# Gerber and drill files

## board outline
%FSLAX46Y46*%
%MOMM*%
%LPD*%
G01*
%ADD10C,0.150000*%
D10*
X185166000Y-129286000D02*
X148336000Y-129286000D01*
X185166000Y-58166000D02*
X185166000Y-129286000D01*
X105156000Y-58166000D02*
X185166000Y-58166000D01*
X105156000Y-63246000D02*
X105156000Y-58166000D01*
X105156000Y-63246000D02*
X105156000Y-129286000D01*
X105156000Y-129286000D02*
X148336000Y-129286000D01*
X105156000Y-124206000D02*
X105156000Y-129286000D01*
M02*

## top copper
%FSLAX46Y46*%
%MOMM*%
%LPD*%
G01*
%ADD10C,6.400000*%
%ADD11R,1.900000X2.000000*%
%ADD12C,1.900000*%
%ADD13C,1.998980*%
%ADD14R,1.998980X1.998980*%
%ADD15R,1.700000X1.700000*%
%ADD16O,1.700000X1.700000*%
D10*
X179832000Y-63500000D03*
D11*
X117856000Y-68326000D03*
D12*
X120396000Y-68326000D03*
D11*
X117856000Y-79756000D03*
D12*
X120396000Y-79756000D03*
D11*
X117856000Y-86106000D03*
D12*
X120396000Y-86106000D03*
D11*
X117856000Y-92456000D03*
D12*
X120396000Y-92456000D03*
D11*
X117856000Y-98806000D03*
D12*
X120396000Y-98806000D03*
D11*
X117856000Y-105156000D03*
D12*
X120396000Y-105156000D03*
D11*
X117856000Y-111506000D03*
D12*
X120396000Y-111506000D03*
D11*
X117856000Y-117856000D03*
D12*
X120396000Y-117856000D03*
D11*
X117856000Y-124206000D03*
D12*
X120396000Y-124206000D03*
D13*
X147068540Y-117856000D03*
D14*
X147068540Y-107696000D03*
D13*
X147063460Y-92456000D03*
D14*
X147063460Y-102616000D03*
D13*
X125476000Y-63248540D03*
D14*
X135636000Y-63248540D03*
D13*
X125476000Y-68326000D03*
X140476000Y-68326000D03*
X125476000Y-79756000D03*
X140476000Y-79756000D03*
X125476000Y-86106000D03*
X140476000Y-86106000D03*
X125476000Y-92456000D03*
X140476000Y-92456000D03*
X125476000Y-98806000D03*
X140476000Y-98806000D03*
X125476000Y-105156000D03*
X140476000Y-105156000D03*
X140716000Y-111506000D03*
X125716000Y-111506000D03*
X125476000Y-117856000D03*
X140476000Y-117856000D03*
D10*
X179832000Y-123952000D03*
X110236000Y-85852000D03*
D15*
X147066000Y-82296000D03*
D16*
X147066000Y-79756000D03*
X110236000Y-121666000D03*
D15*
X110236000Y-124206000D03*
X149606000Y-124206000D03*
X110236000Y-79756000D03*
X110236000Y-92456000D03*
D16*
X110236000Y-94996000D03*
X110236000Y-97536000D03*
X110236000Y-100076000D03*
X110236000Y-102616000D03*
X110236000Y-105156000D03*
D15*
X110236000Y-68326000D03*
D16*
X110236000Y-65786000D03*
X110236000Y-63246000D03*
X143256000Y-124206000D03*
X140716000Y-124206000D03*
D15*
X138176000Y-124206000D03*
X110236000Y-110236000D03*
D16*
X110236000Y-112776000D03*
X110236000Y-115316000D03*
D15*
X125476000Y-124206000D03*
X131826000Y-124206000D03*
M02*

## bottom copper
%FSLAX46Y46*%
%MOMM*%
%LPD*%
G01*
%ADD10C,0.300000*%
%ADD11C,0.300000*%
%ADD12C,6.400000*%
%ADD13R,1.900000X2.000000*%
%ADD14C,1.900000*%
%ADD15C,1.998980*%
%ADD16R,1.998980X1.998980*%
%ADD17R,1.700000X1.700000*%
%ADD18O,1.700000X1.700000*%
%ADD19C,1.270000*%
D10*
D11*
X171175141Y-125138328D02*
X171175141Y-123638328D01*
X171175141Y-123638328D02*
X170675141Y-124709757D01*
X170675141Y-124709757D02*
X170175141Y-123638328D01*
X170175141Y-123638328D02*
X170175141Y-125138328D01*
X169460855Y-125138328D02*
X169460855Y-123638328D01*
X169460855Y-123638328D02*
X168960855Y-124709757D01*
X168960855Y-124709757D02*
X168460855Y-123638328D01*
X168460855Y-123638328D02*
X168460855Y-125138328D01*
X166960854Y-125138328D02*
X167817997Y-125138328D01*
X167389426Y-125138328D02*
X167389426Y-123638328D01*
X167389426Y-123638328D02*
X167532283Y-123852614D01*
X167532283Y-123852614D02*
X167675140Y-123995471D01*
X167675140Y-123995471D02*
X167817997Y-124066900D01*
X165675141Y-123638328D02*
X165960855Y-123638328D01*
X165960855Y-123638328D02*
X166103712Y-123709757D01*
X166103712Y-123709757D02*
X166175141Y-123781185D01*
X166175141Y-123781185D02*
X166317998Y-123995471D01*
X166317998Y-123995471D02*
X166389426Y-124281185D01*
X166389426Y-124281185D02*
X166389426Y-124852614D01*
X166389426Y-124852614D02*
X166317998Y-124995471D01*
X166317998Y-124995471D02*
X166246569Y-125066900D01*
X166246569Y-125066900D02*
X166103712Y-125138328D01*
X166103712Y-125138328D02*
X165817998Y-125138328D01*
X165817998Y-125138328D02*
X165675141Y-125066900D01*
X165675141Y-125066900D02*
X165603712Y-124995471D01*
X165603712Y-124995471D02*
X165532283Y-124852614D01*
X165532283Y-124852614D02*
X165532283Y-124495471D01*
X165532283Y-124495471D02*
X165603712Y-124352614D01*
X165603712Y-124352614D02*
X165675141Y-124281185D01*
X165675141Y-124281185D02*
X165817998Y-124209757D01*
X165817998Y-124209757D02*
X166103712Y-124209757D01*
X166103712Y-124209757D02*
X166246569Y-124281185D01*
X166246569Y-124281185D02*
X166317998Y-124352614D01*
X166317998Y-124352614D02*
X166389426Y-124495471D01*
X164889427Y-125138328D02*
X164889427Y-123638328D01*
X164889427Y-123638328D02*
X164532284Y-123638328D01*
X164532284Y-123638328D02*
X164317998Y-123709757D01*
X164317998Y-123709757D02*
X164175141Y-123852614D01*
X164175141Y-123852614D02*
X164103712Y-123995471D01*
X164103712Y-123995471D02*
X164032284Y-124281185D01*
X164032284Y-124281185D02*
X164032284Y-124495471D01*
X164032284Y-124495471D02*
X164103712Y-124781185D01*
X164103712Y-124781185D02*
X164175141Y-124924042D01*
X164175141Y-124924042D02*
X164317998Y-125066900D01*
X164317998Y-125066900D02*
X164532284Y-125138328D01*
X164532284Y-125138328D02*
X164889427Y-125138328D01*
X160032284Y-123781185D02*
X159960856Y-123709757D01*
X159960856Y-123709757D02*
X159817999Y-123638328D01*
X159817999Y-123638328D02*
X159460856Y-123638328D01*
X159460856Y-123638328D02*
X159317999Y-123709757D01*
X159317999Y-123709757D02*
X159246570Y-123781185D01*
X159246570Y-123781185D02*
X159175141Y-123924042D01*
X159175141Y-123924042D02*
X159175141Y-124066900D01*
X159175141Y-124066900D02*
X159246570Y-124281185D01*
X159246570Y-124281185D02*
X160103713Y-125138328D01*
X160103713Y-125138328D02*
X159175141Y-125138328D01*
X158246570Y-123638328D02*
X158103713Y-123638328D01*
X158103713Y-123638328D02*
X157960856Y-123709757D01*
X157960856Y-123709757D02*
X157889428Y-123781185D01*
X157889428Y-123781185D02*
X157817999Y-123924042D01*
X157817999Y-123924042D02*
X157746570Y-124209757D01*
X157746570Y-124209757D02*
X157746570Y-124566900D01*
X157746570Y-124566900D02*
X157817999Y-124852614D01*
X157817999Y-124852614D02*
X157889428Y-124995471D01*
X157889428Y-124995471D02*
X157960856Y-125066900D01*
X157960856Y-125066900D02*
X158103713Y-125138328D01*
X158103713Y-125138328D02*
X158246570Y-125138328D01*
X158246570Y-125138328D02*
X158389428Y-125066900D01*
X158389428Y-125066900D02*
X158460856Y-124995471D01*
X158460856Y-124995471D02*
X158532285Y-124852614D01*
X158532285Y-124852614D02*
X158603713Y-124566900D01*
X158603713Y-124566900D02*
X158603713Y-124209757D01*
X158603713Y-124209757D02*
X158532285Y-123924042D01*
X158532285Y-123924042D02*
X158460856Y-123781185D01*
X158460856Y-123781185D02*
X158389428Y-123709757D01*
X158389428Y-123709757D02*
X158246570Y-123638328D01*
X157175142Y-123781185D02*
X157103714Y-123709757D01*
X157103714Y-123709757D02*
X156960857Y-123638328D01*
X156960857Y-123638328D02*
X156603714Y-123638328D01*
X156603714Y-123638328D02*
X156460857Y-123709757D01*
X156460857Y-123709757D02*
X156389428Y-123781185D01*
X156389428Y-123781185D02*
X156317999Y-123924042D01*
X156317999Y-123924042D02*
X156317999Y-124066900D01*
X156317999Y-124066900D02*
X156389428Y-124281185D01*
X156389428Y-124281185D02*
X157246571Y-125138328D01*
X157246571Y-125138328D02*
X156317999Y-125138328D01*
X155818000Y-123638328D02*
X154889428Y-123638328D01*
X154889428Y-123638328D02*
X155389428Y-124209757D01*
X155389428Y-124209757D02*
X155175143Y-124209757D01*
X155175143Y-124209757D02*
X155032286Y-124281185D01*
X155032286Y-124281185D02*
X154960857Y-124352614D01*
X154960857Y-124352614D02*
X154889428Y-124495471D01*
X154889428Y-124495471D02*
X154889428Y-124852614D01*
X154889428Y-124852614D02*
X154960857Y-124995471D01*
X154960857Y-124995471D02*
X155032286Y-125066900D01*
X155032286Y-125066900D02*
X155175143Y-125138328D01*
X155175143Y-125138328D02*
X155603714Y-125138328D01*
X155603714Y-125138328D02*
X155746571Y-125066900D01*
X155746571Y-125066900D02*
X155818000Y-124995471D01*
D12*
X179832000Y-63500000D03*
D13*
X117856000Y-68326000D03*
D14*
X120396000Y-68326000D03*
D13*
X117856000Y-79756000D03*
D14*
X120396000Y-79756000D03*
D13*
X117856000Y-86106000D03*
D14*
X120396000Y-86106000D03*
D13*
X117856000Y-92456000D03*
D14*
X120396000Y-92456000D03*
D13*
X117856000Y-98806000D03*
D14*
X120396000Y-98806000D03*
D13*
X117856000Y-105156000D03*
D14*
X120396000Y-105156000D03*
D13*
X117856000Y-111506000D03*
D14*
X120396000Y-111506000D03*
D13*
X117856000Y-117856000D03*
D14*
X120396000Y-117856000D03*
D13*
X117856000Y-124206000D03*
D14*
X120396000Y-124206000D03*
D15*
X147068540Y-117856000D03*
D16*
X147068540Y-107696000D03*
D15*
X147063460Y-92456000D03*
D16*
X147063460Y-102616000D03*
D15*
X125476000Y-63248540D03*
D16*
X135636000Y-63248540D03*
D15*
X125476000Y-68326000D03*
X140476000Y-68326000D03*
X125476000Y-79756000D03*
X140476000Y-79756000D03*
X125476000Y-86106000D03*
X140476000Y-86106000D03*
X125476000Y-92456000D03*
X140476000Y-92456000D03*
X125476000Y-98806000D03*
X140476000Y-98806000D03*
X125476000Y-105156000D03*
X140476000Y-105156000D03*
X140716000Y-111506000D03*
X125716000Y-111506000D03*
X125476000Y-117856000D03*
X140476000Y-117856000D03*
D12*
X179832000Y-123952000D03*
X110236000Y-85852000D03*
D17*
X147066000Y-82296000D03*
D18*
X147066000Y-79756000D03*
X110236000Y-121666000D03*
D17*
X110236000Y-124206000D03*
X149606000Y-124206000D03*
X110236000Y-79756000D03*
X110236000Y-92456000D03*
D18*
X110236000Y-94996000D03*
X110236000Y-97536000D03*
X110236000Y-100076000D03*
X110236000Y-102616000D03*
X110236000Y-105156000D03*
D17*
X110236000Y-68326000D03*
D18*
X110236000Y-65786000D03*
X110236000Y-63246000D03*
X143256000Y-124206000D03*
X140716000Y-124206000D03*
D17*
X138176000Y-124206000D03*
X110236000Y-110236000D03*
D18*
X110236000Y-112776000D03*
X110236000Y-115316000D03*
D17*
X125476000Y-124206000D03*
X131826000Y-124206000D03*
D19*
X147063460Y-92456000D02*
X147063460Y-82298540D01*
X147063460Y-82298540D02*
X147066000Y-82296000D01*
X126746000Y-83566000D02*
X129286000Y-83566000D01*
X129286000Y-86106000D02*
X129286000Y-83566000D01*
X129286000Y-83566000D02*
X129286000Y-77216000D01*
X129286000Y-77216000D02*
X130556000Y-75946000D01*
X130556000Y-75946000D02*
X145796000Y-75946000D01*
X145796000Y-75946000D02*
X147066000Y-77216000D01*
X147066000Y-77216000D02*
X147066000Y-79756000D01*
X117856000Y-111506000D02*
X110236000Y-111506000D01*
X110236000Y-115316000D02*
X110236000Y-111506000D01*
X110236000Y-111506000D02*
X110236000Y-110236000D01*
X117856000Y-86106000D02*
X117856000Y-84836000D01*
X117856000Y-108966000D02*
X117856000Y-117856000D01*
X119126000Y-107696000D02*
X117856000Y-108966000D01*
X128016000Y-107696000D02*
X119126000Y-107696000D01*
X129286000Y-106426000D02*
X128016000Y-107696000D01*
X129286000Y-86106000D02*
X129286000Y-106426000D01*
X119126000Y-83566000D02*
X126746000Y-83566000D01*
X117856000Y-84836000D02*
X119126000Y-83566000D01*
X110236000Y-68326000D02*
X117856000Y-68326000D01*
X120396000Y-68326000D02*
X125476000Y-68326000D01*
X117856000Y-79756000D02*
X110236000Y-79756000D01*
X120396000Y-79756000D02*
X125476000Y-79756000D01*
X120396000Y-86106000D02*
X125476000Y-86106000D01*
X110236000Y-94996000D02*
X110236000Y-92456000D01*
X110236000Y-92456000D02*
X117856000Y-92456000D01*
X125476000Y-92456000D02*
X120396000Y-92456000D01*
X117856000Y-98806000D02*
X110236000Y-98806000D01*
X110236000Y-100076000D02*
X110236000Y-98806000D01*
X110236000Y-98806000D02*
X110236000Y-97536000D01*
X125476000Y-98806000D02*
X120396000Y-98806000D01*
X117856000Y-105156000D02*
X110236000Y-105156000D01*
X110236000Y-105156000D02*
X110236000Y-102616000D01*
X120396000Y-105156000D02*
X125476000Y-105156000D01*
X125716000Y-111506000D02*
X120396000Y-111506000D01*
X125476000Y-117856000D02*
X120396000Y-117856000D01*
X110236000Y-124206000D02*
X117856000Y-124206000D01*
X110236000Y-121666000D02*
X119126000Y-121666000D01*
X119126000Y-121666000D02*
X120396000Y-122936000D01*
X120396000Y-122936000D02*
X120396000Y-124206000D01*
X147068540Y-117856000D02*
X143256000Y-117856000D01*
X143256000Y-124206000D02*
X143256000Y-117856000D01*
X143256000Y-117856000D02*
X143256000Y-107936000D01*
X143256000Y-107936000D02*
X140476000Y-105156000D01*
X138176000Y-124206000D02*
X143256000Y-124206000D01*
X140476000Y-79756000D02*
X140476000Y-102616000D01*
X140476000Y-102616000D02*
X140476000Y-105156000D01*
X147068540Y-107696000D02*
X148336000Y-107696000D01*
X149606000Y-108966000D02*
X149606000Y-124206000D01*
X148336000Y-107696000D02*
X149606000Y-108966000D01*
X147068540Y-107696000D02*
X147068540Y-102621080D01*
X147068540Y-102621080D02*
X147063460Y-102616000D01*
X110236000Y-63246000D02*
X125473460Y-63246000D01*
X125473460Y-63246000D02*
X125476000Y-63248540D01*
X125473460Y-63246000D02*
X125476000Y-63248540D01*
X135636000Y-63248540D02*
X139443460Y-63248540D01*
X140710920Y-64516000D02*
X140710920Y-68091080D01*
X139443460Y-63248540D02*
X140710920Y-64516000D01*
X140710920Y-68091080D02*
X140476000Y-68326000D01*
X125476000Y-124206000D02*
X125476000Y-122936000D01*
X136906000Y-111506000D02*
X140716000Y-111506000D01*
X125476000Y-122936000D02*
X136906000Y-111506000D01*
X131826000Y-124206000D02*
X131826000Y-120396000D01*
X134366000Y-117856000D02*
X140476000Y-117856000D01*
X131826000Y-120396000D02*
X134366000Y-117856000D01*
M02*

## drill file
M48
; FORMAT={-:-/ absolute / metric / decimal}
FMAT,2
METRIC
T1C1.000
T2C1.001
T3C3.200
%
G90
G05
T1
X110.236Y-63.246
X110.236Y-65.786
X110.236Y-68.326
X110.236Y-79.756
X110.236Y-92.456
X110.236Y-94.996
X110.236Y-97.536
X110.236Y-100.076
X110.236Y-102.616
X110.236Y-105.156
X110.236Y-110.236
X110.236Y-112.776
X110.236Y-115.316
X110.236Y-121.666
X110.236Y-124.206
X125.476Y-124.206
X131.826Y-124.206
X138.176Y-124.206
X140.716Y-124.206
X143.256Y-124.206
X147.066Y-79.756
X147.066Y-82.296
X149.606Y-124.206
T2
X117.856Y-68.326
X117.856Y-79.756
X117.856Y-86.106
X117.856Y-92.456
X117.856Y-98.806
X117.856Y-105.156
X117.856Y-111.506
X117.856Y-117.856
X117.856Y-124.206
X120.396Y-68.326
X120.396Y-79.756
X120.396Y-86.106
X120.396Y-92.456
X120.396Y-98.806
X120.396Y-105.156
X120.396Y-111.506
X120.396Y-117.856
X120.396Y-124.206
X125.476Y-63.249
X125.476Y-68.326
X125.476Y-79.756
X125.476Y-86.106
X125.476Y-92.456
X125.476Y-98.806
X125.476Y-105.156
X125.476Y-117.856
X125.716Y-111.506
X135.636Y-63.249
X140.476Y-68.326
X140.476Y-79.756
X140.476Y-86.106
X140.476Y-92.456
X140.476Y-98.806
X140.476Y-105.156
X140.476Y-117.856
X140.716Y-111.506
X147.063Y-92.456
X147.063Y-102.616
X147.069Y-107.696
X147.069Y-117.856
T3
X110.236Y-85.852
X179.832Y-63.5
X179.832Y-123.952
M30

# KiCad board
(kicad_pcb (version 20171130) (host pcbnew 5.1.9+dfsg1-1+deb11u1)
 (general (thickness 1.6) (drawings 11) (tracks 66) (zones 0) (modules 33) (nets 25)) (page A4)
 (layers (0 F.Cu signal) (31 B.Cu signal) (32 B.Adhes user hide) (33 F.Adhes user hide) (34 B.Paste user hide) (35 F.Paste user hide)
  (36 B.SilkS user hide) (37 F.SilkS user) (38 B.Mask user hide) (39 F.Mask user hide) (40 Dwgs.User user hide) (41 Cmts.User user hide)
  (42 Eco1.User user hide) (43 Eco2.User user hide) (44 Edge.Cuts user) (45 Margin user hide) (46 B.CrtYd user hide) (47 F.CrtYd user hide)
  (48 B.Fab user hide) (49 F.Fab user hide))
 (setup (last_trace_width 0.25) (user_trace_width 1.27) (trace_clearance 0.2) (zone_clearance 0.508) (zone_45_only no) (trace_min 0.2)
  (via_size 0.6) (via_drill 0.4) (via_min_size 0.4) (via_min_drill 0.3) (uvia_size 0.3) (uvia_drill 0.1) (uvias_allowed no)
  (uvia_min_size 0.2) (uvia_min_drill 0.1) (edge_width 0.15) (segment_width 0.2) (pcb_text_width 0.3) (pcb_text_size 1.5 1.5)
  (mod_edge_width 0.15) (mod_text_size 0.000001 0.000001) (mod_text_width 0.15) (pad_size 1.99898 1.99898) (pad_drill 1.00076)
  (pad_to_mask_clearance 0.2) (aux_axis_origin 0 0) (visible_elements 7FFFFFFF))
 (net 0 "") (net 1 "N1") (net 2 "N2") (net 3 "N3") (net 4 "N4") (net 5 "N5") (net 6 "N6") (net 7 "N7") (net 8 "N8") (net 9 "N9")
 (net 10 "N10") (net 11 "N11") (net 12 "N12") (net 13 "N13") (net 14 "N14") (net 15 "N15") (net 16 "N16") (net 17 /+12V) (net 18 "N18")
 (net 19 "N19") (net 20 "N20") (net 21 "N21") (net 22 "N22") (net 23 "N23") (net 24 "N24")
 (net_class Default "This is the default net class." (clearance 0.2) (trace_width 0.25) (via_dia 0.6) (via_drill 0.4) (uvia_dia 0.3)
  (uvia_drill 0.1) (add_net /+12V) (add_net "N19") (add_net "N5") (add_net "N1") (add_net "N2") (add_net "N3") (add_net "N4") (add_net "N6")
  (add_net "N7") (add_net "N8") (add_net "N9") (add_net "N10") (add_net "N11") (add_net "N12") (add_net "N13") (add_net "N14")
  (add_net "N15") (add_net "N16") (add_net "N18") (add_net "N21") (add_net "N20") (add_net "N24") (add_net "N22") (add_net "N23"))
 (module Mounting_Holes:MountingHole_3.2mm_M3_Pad (layer F.Cu) (at 179.832 63.5)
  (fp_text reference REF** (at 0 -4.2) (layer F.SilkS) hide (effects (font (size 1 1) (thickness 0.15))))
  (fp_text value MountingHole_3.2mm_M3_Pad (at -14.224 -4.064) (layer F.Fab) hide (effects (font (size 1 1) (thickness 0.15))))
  (pad 1 thru_hole circle (at 0 0) (size 6.4 6.4) (drill 3.2) (layers *.Cu *.Mask)))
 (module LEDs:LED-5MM (layer F.Cu) (at 117.856 68.326)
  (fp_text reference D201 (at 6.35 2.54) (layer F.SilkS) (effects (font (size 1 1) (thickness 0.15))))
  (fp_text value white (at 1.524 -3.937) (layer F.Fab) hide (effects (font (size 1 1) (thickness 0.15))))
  (pad 1 thru_hole rect (at 0 0 90) (size 2 1.9) (drill 1.00076) (layers *.Cu *.Mask) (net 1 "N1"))
  (pad 2 thru_hole circle (at 2.54 0) (size 1.9 1.9) (drill 1.00076) (layers *.Cu *.Mask) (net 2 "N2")))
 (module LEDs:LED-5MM (layer F.Cu) (at 117.856 79.756)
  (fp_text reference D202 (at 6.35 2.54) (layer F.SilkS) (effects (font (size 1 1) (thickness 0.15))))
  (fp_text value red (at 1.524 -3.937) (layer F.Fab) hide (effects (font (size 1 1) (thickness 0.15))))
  (pad 1 thru_hole rect (at 0 0 90) (size 2 1.9) (drill 1.00076) (layers *.Cu *.Mask) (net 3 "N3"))
  (pad 2 thru_hole circle (at 2.54 0) (size 1.9 1.9) (drill 1.00076) (layers *.Cu *.Mask) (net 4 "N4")))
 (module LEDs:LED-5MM (layer F.Cu) (at 117.856 86.106)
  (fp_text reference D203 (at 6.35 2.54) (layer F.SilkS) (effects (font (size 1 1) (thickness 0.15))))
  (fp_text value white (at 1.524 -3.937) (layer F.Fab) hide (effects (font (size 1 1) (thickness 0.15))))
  (pad 1 thru_hole rect (at 0 0 90) (size 2 1.9) (drill 1.00076) (layers *.Cu *.Mask) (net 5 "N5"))
  (pad 2 thru_hole circle (at 2.54 0) (size 1.9 1.9) (drill 1.00076) (layers *.Cu *.Mask) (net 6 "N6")))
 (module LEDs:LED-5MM (layer F.Cu) (at 117.856 92.456)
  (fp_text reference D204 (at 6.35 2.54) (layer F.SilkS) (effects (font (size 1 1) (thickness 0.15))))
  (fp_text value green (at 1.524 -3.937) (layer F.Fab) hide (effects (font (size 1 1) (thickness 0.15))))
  (pad 1 thru_hole rect (at 0 0 90) (size 2 1.9) (drill 1.00076) (layers *.Cu *.Mask) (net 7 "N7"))
  (pad 2 thru_hole circle (at 2.54 0) (size 1.9 1.9) (drill 1.00076) (layers *.Cu *.Mask) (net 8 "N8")))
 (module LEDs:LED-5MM (layer F.Cu) (at 117.856 98.806)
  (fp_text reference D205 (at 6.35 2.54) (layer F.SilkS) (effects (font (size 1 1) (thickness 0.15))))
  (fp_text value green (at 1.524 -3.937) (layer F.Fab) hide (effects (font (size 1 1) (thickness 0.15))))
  (pad 1 thru_hole rect (at 0 0 90) (size 2 1.9) (drill 1.00076) (layers *.Cu *.Mask) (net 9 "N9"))
  (pad 2 thru_hole circle (at 2.54 0) (size 1.9 1.9) (drill 1.00076) (layers *.Cu *.Mask) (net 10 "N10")))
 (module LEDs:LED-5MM (layer F.Cu) (at 117.856 105.156)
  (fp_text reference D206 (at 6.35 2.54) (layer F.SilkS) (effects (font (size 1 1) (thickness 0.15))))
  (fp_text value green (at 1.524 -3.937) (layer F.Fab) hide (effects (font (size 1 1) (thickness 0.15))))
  (pad 1 thru_hole rect (at 0 0 90) (size 2 1.9) (drill 1.00076) (layers *.Cu *.Mask) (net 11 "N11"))
  (pad 2 thru_hole circle (at 2.54 0) (size 1.9 1.9) (drill 1.00076) (layers *.Cu *.Mask) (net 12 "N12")))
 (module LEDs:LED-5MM (layer F.Cu) (at 117.856 111.506)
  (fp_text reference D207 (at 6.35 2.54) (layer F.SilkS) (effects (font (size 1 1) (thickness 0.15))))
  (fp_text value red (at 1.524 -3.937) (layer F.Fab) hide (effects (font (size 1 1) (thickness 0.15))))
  (pad 1 thru_hole rect (at 0 0 90) (size 2 1.9) (drill 1.00076) (layers *.Cu *.Mask) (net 5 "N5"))
  (pad 2 thru_hole circle (at 2.54 0) (size 1.9 1.9) (drill 1.00076) (layers *.Cu *.Mask) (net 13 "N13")))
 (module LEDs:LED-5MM (layer F.Cu) (at 117.856 117.856)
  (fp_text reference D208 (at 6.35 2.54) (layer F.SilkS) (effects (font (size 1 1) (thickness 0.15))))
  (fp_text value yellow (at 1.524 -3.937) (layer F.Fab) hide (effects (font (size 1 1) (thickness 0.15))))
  (pad 1 thru_hole rect (at 0 0 90) (size 2 1.9) (drill 1.00076) (layers *.Cu *.Mask) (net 5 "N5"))
  (pad 2 thru_hole circle (at 2.54 0) (size 1.9 1.9) (drill 1.00076) (layers *.Cu *.Mask) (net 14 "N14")))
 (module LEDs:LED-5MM (layer F.Cu) (at 117.856 124.206)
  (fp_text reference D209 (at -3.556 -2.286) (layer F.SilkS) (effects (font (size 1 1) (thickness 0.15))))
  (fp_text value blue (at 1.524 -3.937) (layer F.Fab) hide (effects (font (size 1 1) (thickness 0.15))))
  (pad 1 thru_hole rect (at 0 0 90) (size 2 1.9) (drill 1.00076) (layers *.Cu *.Mask) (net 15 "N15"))
  (pad 2 thru_hole circle (at 2.54 0) (size 1.9 1.9) (drill 1.00076) (layers *.Cu *.Mask) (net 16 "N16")))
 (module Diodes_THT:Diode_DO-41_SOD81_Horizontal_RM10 (layer F.Cu) (at 147.066 107.696 270)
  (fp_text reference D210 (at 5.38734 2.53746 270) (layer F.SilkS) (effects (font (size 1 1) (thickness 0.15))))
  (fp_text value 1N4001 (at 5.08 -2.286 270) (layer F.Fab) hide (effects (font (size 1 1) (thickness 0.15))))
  (pad 2 thru_hole circle (at 10.16 -0.00254 90) (size 1.99898 1.99898) (drill 1.00076) (layers *.Cu *.Mask) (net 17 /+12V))
  (pad 1 thru_hole rect (at 0 -0.00254 90) (size 1.99898 1.99898) (drill 1.00076) (layers *.Cu *.Mask) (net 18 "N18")))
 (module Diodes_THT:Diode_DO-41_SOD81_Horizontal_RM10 (layer F.Cu) (at 147.066 102.616 90)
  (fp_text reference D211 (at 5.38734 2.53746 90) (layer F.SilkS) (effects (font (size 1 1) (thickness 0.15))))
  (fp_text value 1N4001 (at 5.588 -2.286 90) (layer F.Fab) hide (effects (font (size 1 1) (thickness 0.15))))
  (pad 2 thru_hole circle (at 10.16 -0.00254 270) (size 1.99898 1.99898) (drill 1.00076) (layers *.Cu *.Mask) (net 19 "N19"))
  (pad 1 thru_hole rect (at 0 -0.00254 270) (size 1.99898 1.99898) (drill 1.00076) (layers *.Cu *.Mask) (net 18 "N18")))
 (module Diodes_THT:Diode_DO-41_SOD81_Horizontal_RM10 (layer F.Cu) (at 135.636 63.246 180)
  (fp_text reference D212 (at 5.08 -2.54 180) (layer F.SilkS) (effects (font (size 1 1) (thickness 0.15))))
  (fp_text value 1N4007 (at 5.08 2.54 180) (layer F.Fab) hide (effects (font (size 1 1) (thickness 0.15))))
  (pad 2 thru_hole circle (at 10.16 -0.00254) (size 1.99898 1.99898) (drill 1.00076) (layers *.Cu *.Mask) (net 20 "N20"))
  (pad 1 thru_hole rect (at 0 -0.00254) (size 1.99898 1.99898) (drill 1.00076) (layers *.Cu *.Mask) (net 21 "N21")))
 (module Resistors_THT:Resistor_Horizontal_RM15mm (layer F.Cu) (at 125.476 68.326)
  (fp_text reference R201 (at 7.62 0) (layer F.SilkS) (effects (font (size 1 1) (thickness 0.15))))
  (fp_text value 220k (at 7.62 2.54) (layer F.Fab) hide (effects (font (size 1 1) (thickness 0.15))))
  (pad 1 thru_hole circle (at 0 0) (size 1.99898 1.99898) (drill 1.00076) (layers *.Cu *.SilkS *.Mask) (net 2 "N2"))
  (pad 2 thru_hole circle (at 15 0) (size 1.99898 1.99898) (drill 1.00076) (layers *.Cu *.SilkS *.Mask) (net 21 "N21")))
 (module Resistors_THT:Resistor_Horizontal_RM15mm (layer F.Cu) (at 125.476 79.756)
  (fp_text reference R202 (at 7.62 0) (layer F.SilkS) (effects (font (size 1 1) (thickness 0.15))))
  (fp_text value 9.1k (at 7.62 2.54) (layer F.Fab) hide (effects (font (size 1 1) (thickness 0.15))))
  (pad 1 thru_hole circle (at 0 0) (size 1.99898 1.99898) (drill 1.00076) (layers *.Cu *.SilkS *.Mask) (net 4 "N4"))
  (pad 2 thru_hole circle (at 15 0) (size 1.99898 1.99898) (drill 1.00076) (layers *.Cu *.SilkS *.Mask) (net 17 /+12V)))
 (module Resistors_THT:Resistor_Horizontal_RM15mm (layer F.Cu) (at 125.476 86.106)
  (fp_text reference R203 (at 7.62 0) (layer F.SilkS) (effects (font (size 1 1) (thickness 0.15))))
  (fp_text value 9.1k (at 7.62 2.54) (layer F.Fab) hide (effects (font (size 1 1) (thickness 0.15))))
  (pad 1 thru_hole circle (at 0 0) (size 1.99898 1.99898) (drill 1.00076) (layers *.Cu *.SilkS *.Mask) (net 6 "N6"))
  (pad 2 thru_hole circle (at 15 0) (size 1.99898 1.99898) (drill 1.00076) (layers *.Cu *.SilkS *.Mask) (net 17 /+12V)))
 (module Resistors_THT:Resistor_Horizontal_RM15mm (layer F.Cu) (at 125.476 92.456)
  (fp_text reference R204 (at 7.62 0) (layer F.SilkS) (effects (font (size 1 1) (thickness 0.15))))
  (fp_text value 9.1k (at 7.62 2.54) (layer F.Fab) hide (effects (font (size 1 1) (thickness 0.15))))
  (pad 1 thru_hole circle (at 0 0) (size 1.99898 1.99898) (drill 1.00076) (layers *.Cu *.SilkS *.Mask) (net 8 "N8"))
  (pad 2 thru_hole circle (at 15 0) (size 1.99898 1.99898) (drill 1.00076) (layers *.Cu *.SilkS *.Mask) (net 17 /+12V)))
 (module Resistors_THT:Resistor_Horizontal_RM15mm (layer F.Cu) (at 125.476 98.806)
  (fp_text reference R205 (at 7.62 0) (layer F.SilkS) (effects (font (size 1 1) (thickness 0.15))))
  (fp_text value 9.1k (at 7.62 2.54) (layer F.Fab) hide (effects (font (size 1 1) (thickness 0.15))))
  (pad 1 thru_hole circle (at 0 0) (size 1.99898 1.99898) (drill 1.00076) (layers *.Cu *.SilkS *.Mask) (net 10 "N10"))
  (pad 2 thru_hole circle (at 15 0) (size 1.99898 1.99898) (drill 1.00076) (layers *.Cu *.SilkS *.Mask) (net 17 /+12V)))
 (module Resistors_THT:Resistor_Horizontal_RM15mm (layer F.Cu) (at 125.476 105.156)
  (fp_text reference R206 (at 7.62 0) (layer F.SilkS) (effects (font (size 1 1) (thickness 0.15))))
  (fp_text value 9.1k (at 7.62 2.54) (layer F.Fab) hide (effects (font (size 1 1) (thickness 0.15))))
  (pad 1 thru_hole circle (at 0 0) (size 1.99898 1.99898) (drill 1.00076) (layers *.Cu *.SilkS *.Mask) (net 12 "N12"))
  (pad 2 thru_hole circle (at 15 0) (size 1.99898 1.99898) (drill 1.00076) (layers *.Cu *.SilkS *.Mask) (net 17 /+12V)))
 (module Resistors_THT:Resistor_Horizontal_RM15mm (layer F.Cu) (at 140.716 111.506 180)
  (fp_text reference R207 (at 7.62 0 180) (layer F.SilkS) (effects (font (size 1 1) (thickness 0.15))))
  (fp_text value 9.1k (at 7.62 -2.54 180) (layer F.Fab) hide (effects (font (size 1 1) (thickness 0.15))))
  (pad 1 thru_hole circle (at 0 0 180) (size 1.99898 1.99898) (drill 1.00076) (layers *.Cu *.SilkS *.Mask) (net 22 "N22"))
  (pad 2 thru_hole circle (at 15 0 180) (size 1.99898 1.99898) (drill 1.00076) (layers *.Cu *.SilkS *.Mask) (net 13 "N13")))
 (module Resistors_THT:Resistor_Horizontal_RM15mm (layer F.Cu) (at 125.476 117.856)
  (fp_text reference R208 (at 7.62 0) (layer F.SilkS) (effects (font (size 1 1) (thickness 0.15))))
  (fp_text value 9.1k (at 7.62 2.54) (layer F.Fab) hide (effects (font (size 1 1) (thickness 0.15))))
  (pad 1 thru_hole circle (at 0 0) (size 1.99898 1.99898) (drill 1.00076) (layers *.Cu *.SilkS *.Mask) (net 14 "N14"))
  (pad 2 thru_hole circle (at 15 0) (size 1.99898 1.99898) (drill 1.00076) (layers *.Cu *.SilkS *.Mask) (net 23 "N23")))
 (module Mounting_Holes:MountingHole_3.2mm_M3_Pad (layer F.Cu) (at 179.832 123.952)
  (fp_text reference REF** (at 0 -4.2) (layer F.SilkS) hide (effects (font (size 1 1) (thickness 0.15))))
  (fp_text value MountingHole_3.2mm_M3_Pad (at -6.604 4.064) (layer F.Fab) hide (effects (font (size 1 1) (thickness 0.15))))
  (pad 1 thru_hole circle (at 0 0) (size 6.4 6.4) (drill 3.2) (layers *.Cu *.Mask)))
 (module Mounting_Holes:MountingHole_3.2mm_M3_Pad (layer F.Cu) (at 110.236 85.852)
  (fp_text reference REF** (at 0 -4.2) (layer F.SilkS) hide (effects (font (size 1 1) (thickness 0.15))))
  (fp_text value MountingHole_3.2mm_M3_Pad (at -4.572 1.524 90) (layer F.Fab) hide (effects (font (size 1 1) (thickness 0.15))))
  (pad 1 thru_hole circle (at 0 0) (size 6.4 6.4) (drill 3.2) (layers *.Cu *.Mask)))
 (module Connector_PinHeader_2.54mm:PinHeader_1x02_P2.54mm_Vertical (layer F.Cu) (at 147.066 82.296 180)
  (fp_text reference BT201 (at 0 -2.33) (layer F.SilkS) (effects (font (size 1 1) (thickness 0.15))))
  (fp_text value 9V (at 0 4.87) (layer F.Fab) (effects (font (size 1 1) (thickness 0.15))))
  (pad 1 thru_hole rect (at 0 0 180) (size 1.7 1.7) (drill 1) (layers *.Cu *.Mask) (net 19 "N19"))
  (pad 2 thru_hole oval (at 0 2.54 180) (size 1.7 1.7) (drill 1) (layers *.Cu *.Mask) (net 5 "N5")))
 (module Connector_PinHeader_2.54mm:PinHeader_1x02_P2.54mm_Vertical (layer F.Cu) (at 110.236 124.206 180)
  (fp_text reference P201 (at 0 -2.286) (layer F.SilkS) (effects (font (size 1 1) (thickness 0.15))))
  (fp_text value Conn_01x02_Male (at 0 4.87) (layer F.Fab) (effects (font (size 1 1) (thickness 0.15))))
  (pad 2 thru_hole oval (at 0 2.54 180) (size 1.7 1.7) (drill 1) (layers *.Cu *.Mask) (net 16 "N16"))
  (pad 1 thru_hole rect (at 0 0 180) (size 1.7 1.7) (drill 1) (layers *.Cu *.Mask) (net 15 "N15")))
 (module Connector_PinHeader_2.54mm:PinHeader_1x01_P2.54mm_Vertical (layer F.Cu) (at 149.606 124.206)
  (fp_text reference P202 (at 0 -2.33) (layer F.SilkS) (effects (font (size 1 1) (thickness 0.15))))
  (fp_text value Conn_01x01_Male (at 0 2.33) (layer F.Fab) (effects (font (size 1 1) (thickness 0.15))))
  (pad 1 thru_hole rect (at 0 0) (size 1.7 1.7) (drill 1) (layers *.Cu *.Mask) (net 18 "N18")))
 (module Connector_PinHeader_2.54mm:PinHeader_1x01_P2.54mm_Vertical (layer F.Cu) (at 110.236 79.756 270)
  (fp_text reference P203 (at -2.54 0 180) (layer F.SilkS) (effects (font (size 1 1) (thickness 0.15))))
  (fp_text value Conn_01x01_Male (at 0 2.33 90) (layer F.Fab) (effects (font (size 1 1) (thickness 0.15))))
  (pad 1 thru_hole rect (at 0 0 270) (size 1.7 1.7) (drill 1) (layers *.Cu *.Mask) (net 3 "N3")))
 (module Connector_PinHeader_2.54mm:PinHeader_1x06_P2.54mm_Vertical (layer F.Cu) (at 110.236 92.456)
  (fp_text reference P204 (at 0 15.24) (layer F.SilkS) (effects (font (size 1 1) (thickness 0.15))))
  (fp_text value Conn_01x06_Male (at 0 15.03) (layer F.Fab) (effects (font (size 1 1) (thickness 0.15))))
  (pad 1 thru_hole rect (at 0 0) (size 1.7 1.7) (drill 1) (layers *.Cu *.Mask) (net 7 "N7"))
  (pad 2 thru_hole oval (at 0 2.54) (size 1.7 1.7) (drill 1) (layers *.Cu *.Mask) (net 7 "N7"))
  (pad 3 thru_hole oval (at 0 5.08) (size 1.7 1.7) (drill 1) (layers *.Cu *.Mask) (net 9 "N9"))
  (pad 4 thru_hole oval (at 0 7.62) (size 1.7 1.7) (drill 1) (layers *.Cu *.Mask) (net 9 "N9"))
  (pad 5 thru_hole oval (at 0 10.16) (size 1.7 1.7) (drill 1) (layers *.Cu *.Mask) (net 11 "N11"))
  (pad 6 thru_hole oval (at 0 12.7) (size 1.7 1.7) (drill 1) (layers *.Cu *.Mask) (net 11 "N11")))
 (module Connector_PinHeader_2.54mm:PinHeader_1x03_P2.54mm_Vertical (layer F.Cu) (at 110.236 68.326 180)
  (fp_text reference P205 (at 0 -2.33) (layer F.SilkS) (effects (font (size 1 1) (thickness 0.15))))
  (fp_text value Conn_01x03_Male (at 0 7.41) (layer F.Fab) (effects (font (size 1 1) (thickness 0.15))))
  (pad 1 thru_hole rect (at 0 0 180) (size 1.7 1.7) (drill 1) (layers *.Cu *.Mask) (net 1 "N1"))
  (pad 2 thru_hole oval (at 0 2.54 180) (size 1.7 1.7) (drill 1) (layers *.Cu *.Mask) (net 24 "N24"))
  (pad 3 thru_hole oval (at 0 5.08 180) (size 1.7 1.7) (drill 1) (layers *.Cu *.Mask) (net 20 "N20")))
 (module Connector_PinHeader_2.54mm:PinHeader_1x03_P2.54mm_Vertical (layer F.Cu) (at 138.176 124.206 90)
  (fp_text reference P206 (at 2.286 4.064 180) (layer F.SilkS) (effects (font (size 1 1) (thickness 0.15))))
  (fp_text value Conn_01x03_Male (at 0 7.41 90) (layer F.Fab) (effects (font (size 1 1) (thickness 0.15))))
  (pad 3 thru_hole oval (at 0 5.08 90) (size 1.7 1.7) (drill 1) (layers *.Cu *.Mask) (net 17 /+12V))
  (pad 2 thru_hole oval (at 0 2.54 90) (size 1.7 1.7) (drill 1) (layers *.Cu *.Mask) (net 17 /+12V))
  (pad 1 thru_hole rect (at 0 0 90) (size 1.7 1.7) (drill 1) (layers *.Cu *.Mask) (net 17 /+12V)))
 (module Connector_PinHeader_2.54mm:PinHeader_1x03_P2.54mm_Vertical (layer F.Cu) (at 110.236 110.236)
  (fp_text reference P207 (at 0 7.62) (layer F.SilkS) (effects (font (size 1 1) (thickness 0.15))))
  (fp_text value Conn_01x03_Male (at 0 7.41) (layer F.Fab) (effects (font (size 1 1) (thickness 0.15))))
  (pad 1 thru_hole rect (at 0 0) (size 1.7 1.7) (drill 1) (layers *.Cu *.Mask) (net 5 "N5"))
  (pad 2 thru_hole oval (at 0 2.54) (size 1.7 1.7) (drill 1) (layers *.Cu *.Mask) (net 5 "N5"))
  (pad 3 thru_hole oval (at 0 5.08) (size 1.7 1.7) (drill 1) (layers *.Cu *.Mask) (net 5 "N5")))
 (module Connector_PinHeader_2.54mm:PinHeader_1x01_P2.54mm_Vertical (layer F.Cu) (at 125.476 124.206)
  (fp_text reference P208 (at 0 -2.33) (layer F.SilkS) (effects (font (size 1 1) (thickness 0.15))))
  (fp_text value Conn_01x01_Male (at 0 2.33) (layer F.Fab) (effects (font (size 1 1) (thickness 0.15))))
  (pad 1 thru_hole rect (at 0 0) (size 1.7 1.7) (drill 1) (layers *.Cu *.Mask) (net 22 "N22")))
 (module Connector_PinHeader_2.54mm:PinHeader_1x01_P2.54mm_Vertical (layer F.Cu) (at 131.826 124.206)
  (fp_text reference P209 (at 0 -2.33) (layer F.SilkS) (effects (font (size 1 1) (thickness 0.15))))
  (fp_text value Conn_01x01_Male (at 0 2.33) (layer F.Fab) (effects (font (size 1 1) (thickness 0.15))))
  (pad 1 thru_hole rect (at 0 0) (size 1.7 1.7) (drill 1) (layers *.Cu *.Mask) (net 23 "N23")))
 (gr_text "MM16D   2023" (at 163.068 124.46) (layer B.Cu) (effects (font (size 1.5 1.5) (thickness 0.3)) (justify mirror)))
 (gr_line (start 185.166 129.286) (end 148.336 129.286) (angle 90) (layer Edge.Cuts) (width 0.15))
 (gr_line (start 185.166 58.166) (end 185.166 129.286) (angle 90) (layer Edge.Cuts) (width 0.15))
 (gr_line (start 105.156 58.166) (end 185.166 58.166) (angle 90) (layer Edge.Cuts) (width 0.15))
 (gr_line (start 105.156 63.246) (end 105.156 58.166) (angle 90) (layer Edge.Cuts) (width 0.15))
 (gr_line (start 105.156 63.246) (end 105.156 129.286) (angle 90) (layer Edge.Cuts) (width 0.15))
 (gr_line (start 105.156 129.286) (end 148.336 129.286) (angle 90) (layer Edge.Cuts) (width 0.15))
 (gr_line (start 105.156 124.206) (end 105.156 129.286) (angle 90) (layer Edge.Cuts) (width 0.15))
 (segment (start 147.06346 92.456) (end 147.06346 82.29854) (width 1.27) (layer B.Cu) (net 19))
 (segment (start 147.06346 82.29854) (end 147.066 82.296) (width 1.27) (layer B.Cu) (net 19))
 (segment (start 126.746 83.566) (end 129.286 83.566) (width 1.27) (layer B.Cu) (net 5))
 (segment (start 129.286 86.106) (end 129.286 83.566) (width 1.27) (layer B.Cu) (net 5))
 (segment (start 129.286 83.566) (end 129.286 77.216) (width 1.27) (layer B.Cu) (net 5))
 (segment (start 129.286 77.216) (end 130.556 75.946) (width 1.27) (layer B.Cu) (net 5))
 (segment (start 130.556 75.946) (end 145.796 75.946) (width 1.27) (layer B.Cu) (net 5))
 (segment (start 145.796 75.946) (end 147.066 77.216) (width 1.27) (layer B.Cu) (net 5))
 (segment (start 147.066 77.216) (end 147.066 79.756) (width 1.27) (layer B.Cu) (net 5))
 (segment (start 117.856 111.506) (end 110.236 111.506) (width 1.27) (layer B.Cu) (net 5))
 (segment (start 110.236 115.316) (end 110.236 111.506) (width 1.27) (layer B.Cu) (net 5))
 (segment (start 110.236 111.506) (end 110.236 110.236) (width 1.27) (layer B.Cu) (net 5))
 (segment (start 117.856 86.106) (end 117.856 84.836) (width 1.27) (layer B.Cu) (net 5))
 (segment (start 117.856 108.966) (end 117.856 117.856) (width 1.27) (layer B.Cu) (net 5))
 (segment (start 119.126 107.696) (end 117.856 108.966) (width 1.27) (layer B.Cu) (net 5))
 (segment (start 128.016 107.696) (end 119.126 107.696) (width 1.27) (layer B.Cu) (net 5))
 (segment (start 129.286 106.426) (end 128.016 107.696) (width 1.27) (layer B.Cu) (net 5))
 (segment (start 129.286 86.106) (end 129.286 106.426) (width 1.27) (layer B.Cu) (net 5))
 (segment (start 119.126 83.566) (end 126.746 83.566) (width 1.27) (layer B.Cu) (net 5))
 (segment (start 117.856 84.836) (end 119.126 83.566) (width 1.27) (layer B.Cu) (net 5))
 (segment (start 110.236 68.326) (end 117.856 68.326) (width 1.27) (layer B.Cu) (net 1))
 (segment (start 120.396 68.326) (end 125.476 68.326) (width 1.27) (layer B.Cu) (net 2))
 (segment (start 117.856 79.756) (end 110.236 79.756) (width 1.27) (layer B.Cu) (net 3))
 (segment (start 120.396 79.756) (end 125.476 79.756) (width 1.27) (layer B.Cu) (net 4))
 (segment (start 120.396 86.106) (end 125.476 86.106) (width 1.27) (layer B.Cu) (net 6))
 (segment (start 110.236 94.996) (end 110.236 92.456) (width 1.27) (layer B.Cu) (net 7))
 (segment (start 110.236 92.456) (end 117.856 92.456) (width 1.27) (layer B.Cu) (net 7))
 (segment (start 125.476 92.456) (end 120.396 92.456) (width 1.27) (layer B.Cu) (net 8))
 (segment (start 117.856 98.806) (end 110.236 98.806) (width 1.27) (layer B.Cu) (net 9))
 (segment (start 110.236 100.076) (end 110.236 98.806) (width 1.27) (layer B.Cu) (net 9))
 (segment (start 110.236 98.806) (end 110.236 97.536) (width 1.27) (layer B.Cu) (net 9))
 (segment (start 125.476 98.806) (end 120.396 98.806) (width 1.27) (layer B.Cu) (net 10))
 (segment (start 117.856 105.156) (end 110.236 105.156) (width 1.27) (layer B.Cu) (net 11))
 (segment (start 110.236 105.156) (end 110.236 102.616) (width 1.27) (layer B.Cu) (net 11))
 (segment (start 120.396 105.156) (end 125.476 105.156) (width 1.27) (layer B.Cu) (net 12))
 (segment (start 125.716 111.506) (end 120.396 111.506) (width 1.27) (layer B.Cu) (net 13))
 (segment (start 125.476 117.856) (end 120.396 117.856) (width 1.27) (layer B.Cu) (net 14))
 (segment (start 110.236 124.206) (end 117.856 124.206) (width 1.27) (layer B.Cu) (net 15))
 (segment (start 110.236 121.666) (end 119.126 121.666) (width 1.27) (layer B.Cu) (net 16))
 (segment (start 119.126 121.666) (end 120.396 122.936) (width 1.27) (layer B.Cu) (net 16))
 (segment (start 120.396 122.936) (end 120.396 124.206) (width 1.27) (layer B.Cu) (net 16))
 (segment (start 147.06854 117.856) (end 143.256 117.856) (width 1.27) (layer B.Cu) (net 17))
 (segment (start 143.256 124.206) (end 143.256 117.856) (width 1.27) (layer B.Cu) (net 17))
 (segment (start 143.256 117.856) (end 143.256 107.936) (width 1.27) (layer B.Cu) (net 17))
 (segment (start 143.256 107.936) (end 140.476 105.156) (width 1.27) (layer B.Cu) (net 17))
 (segment (start 138.176 124.206) (end 143.256 124.206) (width 1.27) (layer B.Cu) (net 17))
 (segment (start 140.476 79.756) (end 140.476 102.616) (width 1.27) (layer B.Cu) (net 17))
 (segment (start 140.476 102.616) (end 140.476 105.156) (width 1.27) (layer B.Cu) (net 17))
 (segment (start 147.06854 107.696) (end 148.336 107.696) (width 1.27) (layer B.Cu) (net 18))
 (segment (start 149.606 108.966) (end 149.606 124.206) (width 1.27) (layer B.Cu) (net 18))
 (segment (start 148.336 107.696) (end 149.606 108.966) (width 1.27) (layer B.Cu) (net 18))
 (segment (start 147.06854 107.696) (end 147.06854 102.62108) (width 1.27) (layer B.Cu) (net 18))
 (segment (start 147.06854 102.62108) (end 147.06346 102.616) (width 1.27) (layer B.Cu) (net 18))
 (segment (start 110.236 63.246) (end 125.47346 63.246) (width 1.27) (layer B.Cu) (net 20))
 (segment (start 125.47346 63.246) (end 125.476 63.24854) (width 1.27) (layer B.Cu) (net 20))
 (segment (start 125.47346 63.246) (end 125.476 63.24854) (width 1.27) (layer B.Cu) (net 20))
 (segment (start 135.636 63.24854) (end 139.44346 63.24854) (width 1.27) (layer B.Cu) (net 21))
 (segment (start 140.71092 64.516) (end 140.71092 68.09108) (width 1.27) (layer B.Cu) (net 21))
 (segment (start 139.44346 63.24854) (end 140.71092 64.516) (width 1.27) (layer B.Cu) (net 21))
 (segment (start 140.71092 68.09108) (end 140.476 68.326) (width 1.27) (layer B.Cu) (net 21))
 (segment (start 125.476 124.206) (end 125.476 122.936) (width 1.27) (layer B.Cu) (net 22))
 (segment (start 136.906 111.506) (end 140.716 111.506) (width 1.27) (layer B.Cu) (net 22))
 (segment (start 125.476 122.936) (end 136.906 111.506) (width 1.27) (layer B.Cu) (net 22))
 (segment (start 131.826 124.206) (end 131.826 120.396) (width 1.27) (layer B.Cu) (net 23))
 (segment (start 134.366 117.856) (end 140.476 117.856) (width 1.27) (layer B.Cu) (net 23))
 (segment (start 131.826 120.396) (end 134.366 117.856) (width 1.27) (layer B.Cu) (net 23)))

